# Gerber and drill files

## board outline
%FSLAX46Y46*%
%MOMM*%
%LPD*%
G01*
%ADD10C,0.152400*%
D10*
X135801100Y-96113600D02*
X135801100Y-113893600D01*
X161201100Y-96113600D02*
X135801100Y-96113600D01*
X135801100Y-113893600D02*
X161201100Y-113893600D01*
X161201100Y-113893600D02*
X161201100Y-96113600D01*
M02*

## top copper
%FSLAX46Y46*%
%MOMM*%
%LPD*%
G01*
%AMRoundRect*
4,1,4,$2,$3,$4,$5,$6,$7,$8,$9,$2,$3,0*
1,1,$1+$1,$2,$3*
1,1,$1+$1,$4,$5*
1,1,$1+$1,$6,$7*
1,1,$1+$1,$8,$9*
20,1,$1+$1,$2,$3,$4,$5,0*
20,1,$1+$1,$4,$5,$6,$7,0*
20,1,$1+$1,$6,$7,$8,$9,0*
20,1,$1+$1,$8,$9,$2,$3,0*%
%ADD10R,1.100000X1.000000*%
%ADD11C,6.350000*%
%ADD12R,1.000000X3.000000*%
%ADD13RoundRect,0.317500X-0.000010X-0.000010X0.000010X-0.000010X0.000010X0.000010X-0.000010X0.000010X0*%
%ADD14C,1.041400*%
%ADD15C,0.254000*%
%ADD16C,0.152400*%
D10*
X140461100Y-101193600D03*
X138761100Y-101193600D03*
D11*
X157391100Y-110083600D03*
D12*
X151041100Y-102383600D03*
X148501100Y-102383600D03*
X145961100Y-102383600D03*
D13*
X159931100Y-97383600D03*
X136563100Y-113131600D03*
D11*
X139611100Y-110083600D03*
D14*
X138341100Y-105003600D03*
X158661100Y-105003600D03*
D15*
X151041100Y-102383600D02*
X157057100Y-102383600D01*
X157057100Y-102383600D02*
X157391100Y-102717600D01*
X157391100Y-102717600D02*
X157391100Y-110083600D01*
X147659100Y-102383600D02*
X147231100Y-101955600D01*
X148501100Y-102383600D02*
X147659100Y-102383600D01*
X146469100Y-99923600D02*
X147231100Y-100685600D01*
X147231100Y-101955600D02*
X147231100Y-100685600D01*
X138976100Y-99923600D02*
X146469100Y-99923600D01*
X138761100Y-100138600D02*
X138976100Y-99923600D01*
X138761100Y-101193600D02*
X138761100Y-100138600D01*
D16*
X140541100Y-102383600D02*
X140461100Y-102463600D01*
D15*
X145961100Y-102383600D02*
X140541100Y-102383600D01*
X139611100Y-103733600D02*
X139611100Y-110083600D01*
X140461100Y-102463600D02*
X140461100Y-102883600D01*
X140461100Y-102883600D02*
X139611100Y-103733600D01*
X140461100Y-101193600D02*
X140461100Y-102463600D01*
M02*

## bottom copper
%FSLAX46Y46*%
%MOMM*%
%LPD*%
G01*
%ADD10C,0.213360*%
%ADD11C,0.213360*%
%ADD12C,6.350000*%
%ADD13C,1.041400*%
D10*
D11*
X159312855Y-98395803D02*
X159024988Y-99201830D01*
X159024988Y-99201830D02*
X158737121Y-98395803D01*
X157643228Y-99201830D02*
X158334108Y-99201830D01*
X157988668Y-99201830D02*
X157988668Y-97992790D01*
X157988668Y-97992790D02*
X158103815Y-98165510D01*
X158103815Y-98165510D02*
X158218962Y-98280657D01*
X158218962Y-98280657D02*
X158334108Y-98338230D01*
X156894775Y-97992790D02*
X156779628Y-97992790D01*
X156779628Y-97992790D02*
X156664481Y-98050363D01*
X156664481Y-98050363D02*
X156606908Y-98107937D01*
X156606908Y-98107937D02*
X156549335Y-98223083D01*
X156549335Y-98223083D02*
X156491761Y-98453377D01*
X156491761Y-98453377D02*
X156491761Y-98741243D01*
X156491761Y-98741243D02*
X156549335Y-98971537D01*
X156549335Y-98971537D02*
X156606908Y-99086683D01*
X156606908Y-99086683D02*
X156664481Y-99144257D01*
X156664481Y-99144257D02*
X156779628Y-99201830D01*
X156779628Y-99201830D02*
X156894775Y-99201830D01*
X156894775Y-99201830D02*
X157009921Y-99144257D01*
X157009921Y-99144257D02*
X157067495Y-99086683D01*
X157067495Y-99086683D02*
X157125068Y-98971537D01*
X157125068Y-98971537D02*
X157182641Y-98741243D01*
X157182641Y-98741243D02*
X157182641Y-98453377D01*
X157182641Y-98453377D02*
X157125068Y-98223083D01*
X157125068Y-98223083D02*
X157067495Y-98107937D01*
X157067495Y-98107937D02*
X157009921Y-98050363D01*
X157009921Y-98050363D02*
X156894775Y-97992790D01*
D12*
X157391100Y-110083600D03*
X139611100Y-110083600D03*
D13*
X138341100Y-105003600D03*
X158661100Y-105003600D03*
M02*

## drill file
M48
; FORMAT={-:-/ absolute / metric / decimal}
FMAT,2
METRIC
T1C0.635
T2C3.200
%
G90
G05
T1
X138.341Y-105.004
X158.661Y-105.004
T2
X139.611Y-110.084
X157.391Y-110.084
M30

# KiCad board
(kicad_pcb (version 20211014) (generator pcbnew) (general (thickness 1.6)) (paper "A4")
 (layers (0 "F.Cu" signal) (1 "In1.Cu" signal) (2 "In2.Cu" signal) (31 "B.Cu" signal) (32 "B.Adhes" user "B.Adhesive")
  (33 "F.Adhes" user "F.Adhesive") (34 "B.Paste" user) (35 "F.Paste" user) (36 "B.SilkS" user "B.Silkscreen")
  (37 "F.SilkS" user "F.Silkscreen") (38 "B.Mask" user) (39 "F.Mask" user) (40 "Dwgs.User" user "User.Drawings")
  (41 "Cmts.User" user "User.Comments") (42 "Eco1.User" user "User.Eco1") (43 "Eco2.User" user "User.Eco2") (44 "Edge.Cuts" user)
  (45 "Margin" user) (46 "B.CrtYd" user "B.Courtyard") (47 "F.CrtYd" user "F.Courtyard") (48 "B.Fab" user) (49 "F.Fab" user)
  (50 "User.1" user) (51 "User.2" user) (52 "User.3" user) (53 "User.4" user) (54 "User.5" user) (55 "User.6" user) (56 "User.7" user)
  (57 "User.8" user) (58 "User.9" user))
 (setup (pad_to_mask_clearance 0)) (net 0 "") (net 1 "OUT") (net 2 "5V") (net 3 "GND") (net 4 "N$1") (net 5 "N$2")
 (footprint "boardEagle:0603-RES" (layer "F.Cu") (at 139.6111 101.1936 180)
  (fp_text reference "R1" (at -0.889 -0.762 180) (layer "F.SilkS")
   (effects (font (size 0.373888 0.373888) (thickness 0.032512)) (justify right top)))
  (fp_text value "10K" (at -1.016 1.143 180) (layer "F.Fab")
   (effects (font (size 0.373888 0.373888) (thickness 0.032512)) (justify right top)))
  (pad "1" smd rect (at -0.85 0 180) (size 1.1 1) (layers "F.Cu" "F.Paste" "F.Mask") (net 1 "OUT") (solder_mask_margin 0.1016))
  (pad "2" smd rect (at 0.85 0 180) (size 1.1 1) (layers "F.Cu" "F.Paste" "F.Mask") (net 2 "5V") (solder_mask_margin 0.1016)))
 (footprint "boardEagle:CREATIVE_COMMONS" (layer "F.Cu") (at 58.3311 98.6536)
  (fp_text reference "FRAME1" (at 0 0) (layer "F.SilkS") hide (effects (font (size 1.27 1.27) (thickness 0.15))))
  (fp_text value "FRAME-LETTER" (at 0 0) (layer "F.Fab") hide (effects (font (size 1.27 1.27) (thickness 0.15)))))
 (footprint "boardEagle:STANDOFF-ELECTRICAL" (layer "F.Cu") (at 157.3911 110.0836)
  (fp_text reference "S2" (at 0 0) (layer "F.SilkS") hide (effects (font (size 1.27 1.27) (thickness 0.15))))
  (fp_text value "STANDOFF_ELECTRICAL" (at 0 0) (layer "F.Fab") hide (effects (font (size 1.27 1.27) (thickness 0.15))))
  (pad "P1" thru_hole circle (at 0 0) (size 6.35 6.35) (drill 3.2) (layers *.Cu *.Mask) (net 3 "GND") (solder_mask_margin 0.1016)))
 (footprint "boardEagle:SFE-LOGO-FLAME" (layer "F.Cu") (at 157.3911 99.9236)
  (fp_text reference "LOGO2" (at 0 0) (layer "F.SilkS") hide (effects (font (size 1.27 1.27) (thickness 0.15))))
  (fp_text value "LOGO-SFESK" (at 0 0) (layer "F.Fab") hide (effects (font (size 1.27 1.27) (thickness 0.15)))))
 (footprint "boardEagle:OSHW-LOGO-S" (layer "F.Cu") (at 154.8511 98.6536)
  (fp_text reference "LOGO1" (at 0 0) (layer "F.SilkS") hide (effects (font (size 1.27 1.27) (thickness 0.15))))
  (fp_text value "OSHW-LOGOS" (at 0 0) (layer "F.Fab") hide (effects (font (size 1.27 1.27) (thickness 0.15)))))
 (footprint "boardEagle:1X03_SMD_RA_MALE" (layer "F.Cu") (at 148.5011 97.3836 180)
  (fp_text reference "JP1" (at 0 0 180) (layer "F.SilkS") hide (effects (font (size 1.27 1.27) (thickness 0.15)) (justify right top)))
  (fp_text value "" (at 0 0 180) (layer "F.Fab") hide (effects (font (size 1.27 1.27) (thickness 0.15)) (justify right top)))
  (pad "1" smd rect (at -2.54 -5 270) (size 3 1) (layers "F.Cu" "F.Paste" "F.Mask") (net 3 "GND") (solder_mask_margin 0.1016))
  (pad "2" smd rect (at 0 -5 270) (size 3 1) (layers "F.Cu" "F.Paste" "F.Mask") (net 2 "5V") (solder_mask_margin 0.1016))
  (pad "3" smd rect (at 2.54 -5 270) (size 3 1) (layers "F.Cu" "F.Paste" "F.Mask") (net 1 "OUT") (solder_mask_margin 0.1016)))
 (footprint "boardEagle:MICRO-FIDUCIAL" (layer "F.Cu") (at 159.9311 97.3836)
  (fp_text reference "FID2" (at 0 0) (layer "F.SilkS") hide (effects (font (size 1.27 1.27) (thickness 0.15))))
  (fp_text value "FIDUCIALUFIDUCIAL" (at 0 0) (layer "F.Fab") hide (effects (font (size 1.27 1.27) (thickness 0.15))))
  (pad "1" smd roundrect (at 0 0) (size 0.635 0.635) (layers "F.Cu" "F.Mask") (roundrect_rratio 0.5) (solder_mask_margin 0.1016)))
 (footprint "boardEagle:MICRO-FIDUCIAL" (layer "F.Cu") (at 136.5631 113.1316)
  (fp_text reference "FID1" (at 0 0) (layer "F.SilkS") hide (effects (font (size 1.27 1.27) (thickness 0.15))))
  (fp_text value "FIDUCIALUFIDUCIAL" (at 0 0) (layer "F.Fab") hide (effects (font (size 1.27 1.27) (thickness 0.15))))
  (pad "1" smd roundrect (at 0 0) (size 0.635 0.635) (layers "F.Cu" "F.Mask") (roundrect_rratio 0.5) (solder_mask_margin 0.1016)))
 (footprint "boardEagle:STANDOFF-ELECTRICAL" (layer "F.Cu") (at 139.6111 110.0836)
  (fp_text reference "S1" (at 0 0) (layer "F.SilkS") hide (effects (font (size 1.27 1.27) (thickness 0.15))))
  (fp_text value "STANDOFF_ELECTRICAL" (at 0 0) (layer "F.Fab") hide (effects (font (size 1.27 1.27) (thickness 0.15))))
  (pad "P1" thru_hole circle (at 0 0) (size 6.35 6.35) (drill 3.2) (layers *.Cu *.Mask) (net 1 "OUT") (solder_mask_margin 0.1016)))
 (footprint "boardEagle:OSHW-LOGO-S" (layer "B.Cu") (at 142.1511 98.6536 180)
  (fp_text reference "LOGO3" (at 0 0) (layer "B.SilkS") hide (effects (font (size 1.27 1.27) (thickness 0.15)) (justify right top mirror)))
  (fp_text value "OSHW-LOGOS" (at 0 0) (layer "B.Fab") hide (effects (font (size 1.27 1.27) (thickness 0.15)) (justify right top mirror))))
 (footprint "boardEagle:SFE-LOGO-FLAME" (layer "B.Cu") (at 139.6111 99.9236 180)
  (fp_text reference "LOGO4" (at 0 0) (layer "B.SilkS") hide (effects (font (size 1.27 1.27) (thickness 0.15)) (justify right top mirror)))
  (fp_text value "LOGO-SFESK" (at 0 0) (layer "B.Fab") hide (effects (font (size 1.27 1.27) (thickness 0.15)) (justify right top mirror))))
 (gr_line (start 135.8011 96.1136) (end 135.8011 113.8936) (layer "Edge.Cuts") (width 0.1524))
 (gr_line (start 161.2011 96.1136) (end 135.8011 96.1136) (layer "Edge.Cuts") (width 0.1524))
 (gr_line (start 135.8011 113.8936) (end 161.2011 113.8936) (layer "Edge.Cuts") (width 0.1524))
 (gr_line (start 161.2011 113.8936) (end 161.2011 96.1136) (layer "Edge.Cuts") (width 0.1524))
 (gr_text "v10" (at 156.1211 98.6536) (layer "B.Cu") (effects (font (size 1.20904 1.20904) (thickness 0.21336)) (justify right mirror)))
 (segment (start 151.0411 102.3836) (end 157.0571 102.3836) (width 0.254) (layer "F.Cu") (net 3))
 (segment (start 157.0571 102.3836) (end 157.3911 102.7176) (width 0.254) (layer "F.Cu") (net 3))
 (segment (start 157.3911 102.7176) (end 157.3911 110.0836) (width 0.254) (layer "F.Cu") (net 3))
 (segment (start 147.6591 102.3836) (end 147.2311 101.9556) (width 0.254) (layer "F.Cu") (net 2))
 (segment (start 148.5011 102.3836) (end 147.6591 102.3836) (width 0.254) (layer "F.Cu") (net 2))
 (segment (start 146.4691 99.9236) (end 147.2311 100.6856) (width 0.254) (layer "F.Cu") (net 2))
 (segment (start 147.2311 101.9556) (end 147.2311 100.6856) (width 0.254) (layer "F.Cu") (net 2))
 (segment (start 138.9761 99.9236) (end 146.4691 99.9236) (width 0.254) (layer "F.Cu") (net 2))
 (segment (start 138.7611 100.1386) (end 138.9761 99.9236) (width 0.254) (layer "F.Cu") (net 2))
 (segment (start 138.7611 101.1936) (end 138.7611 100.1386) (width 0.254) (layer "F.Cu") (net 2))
 (segment (start 140.5411 102.3836) (end 140.4611 102.4636) (width 0.1524) (layer "F.Cu") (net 1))
 (segment (start 145.9611 102.3836) (end 140.5411 102.3836) (width 0.254) (layer "F.Cu") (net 1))
 (segment (start 139.6111 103.7336) (end 139.6111 110.0836) (width 0.254) (layer "F.Cu") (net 1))
 (segment (start 140.4611 102.4636) (end 140.4611 102.8836) (width 0.254) (layer "F.Cu") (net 1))
 (segment (start 140.4611 102.8836) (end 139.6111 103.7336) (width 0.254) (layer "F.Cu") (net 1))
 (segment (start 140.4611 101.1936) (end 140.4611 102.4636) (width 0.254) (layer "F.Cu") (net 1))
 (via (at 138.3411 105.0036) (size 1.0414) (drill 0.635) (layers "F.Cu" "B.Cu") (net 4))
 (via (at 158.6611 105.0036) (size 1.0414) (drill 0.635) (layers "F.Cu" "B.Cu") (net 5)))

